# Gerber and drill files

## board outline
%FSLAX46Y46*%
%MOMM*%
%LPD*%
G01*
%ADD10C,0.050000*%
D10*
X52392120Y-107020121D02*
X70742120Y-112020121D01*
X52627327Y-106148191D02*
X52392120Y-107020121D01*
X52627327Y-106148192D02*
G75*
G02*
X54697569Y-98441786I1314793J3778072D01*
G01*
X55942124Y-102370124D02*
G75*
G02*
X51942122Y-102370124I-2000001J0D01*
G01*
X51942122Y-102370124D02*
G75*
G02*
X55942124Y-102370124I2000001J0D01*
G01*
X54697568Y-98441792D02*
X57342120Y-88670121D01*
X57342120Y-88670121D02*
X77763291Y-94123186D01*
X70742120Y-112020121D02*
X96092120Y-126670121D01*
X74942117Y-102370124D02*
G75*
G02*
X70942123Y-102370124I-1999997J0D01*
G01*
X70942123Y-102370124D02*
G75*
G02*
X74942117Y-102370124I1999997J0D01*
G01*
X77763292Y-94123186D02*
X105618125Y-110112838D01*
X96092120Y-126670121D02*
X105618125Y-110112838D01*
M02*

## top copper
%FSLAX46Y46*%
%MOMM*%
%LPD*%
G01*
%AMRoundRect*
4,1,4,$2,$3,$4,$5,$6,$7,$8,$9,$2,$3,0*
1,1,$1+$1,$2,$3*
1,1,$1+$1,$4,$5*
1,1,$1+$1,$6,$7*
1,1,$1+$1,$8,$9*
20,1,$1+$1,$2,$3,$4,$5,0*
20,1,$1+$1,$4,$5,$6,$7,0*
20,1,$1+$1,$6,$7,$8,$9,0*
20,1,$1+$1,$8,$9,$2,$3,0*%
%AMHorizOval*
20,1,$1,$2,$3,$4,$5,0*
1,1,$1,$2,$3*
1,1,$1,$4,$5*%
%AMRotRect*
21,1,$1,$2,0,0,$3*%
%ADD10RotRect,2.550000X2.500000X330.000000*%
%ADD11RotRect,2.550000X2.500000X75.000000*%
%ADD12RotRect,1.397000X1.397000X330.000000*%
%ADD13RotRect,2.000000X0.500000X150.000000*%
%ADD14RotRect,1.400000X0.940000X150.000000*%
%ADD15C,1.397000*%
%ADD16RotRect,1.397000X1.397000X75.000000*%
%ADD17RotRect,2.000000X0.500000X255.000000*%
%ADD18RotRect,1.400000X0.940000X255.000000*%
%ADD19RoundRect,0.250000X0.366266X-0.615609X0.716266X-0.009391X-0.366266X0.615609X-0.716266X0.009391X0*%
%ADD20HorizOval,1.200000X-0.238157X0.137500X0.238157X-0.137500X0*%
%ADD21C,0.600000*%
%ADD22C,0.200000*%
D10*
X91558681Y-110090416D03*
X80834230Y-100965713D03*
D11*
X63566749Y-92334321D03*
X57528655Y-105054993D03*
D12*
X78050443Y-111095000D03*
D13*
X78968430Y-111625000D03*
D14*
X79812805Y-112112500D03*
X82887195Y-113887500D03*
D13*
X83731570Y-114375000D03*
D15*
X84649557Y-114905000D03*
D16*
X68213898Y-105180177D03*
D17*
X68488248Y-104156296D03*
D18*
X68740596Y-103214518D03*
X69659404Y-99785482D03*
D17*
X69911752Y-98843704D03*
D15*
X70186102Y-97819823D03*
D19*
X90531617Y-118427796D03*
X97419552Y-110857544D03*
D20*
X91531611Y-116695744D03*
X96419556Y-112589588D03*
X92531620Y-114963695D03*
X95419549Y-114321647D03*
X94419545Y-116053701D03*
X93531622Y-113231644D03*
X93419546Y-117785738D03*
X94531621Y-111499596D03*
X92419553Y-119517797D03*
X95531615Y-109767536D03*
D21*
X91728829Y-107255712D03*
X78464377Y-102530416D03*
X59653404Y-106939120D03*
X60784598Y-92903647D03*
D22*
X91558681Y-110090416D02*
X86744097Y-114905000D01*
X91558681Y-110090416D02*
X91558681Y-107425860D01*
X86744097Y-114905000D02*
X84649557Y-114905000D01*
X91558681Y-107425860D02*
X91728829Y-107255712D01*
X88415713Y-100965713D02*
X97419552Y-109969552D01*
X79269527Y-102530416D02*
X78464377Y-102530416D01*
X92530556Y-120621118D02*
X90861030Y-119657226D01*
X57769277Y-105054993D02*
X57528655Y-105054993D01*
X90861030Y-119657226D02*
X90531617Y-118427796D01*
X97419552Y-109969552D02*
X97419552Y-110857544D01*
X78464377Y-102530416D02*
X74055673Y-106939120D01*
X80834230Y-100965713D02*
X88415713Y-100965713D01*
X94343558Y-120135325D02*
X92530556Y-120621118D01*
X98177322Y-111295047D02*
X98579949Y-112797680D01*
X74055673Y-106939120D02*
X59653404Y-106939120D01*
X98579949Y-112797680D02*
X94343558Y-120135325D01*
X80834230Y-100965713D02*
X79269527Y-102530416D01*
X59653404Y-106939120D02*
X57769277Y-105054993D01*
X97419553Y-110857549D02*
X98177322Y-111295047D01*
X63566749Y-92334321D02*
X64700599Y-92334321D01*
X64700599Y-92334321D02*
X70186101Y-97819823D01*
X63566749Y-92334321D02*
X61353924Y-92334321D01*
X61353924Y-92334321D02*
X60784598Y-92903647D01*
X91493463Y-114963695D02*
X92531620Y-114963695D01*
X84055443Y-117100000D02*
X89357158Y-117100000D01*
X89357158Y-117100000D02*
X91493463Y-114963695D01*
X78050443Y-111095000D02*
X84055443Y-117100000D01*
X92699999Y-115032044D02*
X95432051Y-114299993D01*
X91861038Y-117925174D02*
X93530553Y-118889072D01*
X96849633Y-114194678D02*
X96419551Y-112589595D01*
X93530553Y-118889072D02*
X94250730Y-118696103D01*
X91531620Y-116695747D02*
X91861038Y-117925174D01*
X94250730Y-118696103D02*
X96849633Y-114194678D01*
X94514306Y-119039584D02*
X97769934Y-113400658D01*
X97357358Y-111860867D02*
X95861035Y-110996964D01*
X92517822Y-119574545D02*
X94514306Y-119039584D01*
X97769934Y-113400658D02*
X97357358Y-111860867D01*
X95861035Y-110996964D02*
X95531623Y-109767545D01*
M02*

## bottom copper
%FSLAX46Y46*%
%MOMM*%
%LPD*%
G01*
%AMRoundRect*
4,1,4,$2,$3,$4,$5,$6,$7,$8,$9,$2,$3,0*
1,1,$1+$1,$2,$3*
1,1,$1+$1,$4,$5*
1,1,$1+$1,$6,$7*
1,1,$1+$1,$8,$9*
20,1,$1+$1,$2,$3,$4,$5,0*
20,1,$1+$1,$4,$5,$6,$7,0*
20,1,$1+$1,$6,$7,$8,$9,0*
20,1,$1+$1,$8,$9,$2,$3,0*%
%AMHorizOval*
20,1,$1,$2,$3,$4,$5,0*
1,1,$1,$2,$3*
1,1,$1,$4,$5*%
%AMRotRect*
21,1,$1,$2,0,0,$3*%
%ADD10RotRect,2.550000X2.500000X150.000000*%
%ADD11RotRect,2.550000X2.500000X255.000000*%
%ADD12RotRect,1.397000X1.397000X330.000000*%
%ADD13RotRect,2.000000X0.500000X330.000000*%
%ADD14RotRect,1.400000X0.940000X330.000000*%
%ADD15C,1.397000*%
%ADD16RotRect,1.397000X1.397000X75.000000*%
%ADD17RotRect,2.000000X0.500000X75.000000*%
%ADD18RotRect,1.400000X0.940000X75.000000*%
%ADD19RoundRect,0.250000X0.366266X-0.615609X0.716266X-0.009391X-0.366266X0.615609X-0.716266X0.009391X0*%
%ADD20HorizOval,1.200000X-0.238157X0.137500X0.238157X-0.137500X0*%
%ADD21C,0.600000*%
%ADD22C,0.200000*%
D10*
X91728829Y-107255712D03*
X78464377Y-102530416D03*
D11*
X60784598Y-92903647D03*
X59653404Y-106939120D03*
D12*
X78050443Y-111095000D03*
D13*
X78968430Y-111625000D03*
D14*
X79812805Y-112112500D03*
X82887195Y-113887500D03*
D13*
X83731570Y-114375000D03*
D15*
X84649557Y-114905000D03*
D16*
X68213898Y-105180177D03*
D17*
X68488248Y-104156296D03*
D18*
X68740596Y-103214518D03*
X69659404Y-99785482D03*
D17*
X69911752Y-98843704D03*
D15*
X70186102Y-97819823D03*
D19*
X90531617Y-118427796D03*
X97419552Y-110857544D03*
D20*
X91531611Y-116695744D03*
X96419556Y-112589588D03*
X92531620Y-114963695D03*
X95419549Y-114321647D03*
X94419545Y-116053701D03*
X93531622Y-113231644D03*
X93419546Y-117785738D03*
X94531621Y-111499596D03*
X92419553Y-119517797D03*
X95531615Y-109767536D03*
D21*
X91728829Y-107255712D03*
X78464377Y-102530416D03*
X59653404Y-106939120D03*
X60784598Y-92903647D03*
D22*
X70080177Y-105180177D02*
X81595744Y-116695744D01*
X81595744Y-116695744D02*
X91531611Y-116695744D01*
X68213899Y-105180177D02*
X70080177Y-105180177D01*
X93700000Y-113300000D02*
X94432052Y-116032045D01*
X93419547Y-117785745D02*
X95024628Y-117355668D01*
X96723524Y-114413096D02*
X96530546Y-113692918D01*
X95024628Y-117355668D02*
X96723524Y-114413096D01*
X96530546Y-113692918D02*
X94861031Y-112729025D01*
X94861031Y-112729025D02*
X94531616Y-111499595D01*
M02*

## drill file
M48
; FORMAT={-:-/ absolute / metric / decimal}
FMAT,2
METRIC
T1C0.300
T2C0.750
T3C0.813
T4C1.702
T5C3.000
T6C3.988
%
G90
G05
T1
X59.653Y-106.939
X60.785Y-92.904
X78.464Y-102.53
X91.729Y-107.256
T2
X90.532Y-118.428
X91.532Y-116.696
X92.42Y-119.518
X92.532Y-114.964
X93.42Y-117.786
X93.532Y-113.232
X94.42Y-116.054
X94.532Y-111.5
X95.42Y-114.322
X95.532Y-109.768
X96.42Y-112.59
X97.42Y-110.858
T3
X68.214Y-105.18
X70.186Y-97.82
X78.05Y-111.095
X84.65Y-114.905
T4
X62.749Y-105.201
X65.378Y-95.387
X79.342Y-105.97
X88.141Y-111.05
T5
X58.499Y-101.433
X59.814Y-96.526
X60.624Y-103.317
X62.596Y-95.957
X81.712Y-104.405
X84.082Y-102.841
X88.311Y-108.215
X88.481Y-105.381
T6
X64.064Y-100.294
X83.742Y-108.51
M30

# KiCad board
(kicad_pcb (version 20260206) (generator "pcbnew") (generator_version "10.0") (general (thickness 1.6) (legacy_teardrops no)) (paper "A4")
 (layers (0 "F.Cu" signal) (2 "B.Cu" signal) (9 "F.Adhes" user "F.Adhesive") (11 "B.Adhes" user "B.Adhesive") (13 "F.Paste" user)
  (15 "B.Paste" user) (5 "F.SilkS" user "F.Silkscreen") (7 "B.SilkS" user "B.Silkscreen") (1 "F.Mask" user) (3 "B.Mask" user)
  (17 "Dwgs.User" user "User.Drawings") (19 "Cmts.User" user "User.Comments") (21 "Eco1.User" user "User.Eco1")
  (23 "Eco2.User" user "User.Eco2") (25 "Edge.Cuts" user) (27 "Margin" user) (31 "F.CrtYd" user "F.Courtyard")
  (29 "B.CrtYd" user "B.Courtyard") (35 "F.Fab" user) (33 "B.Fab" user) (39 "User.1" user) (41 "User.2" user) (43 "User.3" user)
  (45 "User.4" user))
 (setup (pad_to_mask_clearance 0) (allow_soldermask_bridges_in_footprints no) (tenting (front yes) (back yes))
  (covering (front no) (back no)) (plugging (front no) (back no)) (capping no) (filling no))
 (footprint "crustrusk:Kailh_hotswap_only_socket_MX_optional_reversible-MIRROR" (layer "F.Cu") (at 83.741529 108.510121 -30)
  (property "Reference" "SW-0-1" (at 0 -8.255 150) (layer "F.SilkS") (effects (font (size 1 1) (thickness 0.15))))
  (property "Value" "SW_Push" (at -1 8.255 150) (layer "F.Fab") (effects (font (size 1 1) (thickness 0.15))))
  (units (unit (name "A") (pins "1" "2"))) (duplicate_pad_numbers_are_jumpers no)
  (pad "" np_thru_hole circle (at -5.08 0 330) (size 1.7018 1.7018) (drill 1.7018) (layers "*.Cu" "*.Mask"))
  (pad "" np_thru_hole circle (at -3.81 -2.54 150) (size 3 3) (drill 3) (layers "*.Cu" "*.Mask"))
  (pad "" np_thru_hole circle (at -2.54 -5.079997 330) (size 3 3) (drill 3) (layers "*.Cu" "*.Mask"))
  (pad "" np_thru_hole circle (at 0 0 330) (size 3.9878 3.9878) (drill 3.9878) (layers "*.Cu" "*.Mask"))
  (pad "" np_thru_hole circle (at 2.540002 -5.080001 150) (size 3 3) (drill 3) (layers "*.Cu" "*.Mask"))
  (pad "" np_thru_hole circle (at 3.81 -2.540001 330) (size 3 3) (drill 3) (layers "*.Cu" "*.Mask"))
  (pad "" np_thru_hole circle (at 5.08 0 330) (size 1.7018 1.7018) (drill 1.7018) (layers "*.Cu" "*.Mask"))
  (pad "1" smd rect (at 6.29 -5.08 150) (size 2.55 2.5) (layers "B.Cu" "B.Mask" "B.Paste") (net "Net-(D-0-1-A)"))
  (pad "1" smd rect (at 7.56 -2.54 330) (size 2.55 2.5) (layers "F.Cu" "F.Mask" "F.Paste") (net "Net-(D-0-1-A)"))
  (pad "2" smd rect (at -7.56 -2.54 150) (size 2.55 2.5) (layers "B.Cu" "B.Mask" "B.Paste") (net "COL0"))
  (pad "2" smd rect (at -6.289999 -5.079999 330) (size 2.55 2.5) (layers "F.Cu" "F.Mask" "F.Paste") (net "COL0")))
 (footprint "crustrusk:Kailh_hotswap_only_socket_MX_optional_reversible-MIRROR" (layer "F.Cu") (at 64.063529 100.294121 75)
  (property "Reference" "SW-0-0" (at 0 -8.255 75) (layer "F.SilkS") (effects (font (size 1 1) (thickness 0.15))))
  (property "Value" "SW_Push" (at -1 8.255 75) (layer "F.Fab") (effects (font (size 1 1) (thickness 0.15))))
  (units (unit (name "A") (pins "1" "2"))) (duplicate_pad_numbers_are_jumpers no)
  (pad "" np_thru_hole circle (at -5.08 0 75) (size 1.7018 1.7018) (drill 1.7018) (layers "*.Cu" "*.Mask"))
  (pad "" np_thru_hole circle (at -3.810001 -2.54 255) (size 3 3) (drill 3) (layers "*.Cu" "*.Mask"))
  (pad "" np_thru_hole circle (at -2.54 -5.079998 75) (size 3 3) (drill 3) (layers "*.Cu" "*.Mask"))
  (pad "" np_thru_hole circle (at 0 0 75) (size 3.9878 3.9878) (drill 3.9878) (layers "*.Cu" "*.Mask"))
  (pad "" np_thru_hole circle (at 2.540003 -5.080001 255) (size 3 3) (drill 3) (layers "*.Cu" "*.Mask"))
  (pad "" np_thru_hole circle (at 3.81 -2.54 75) (size 3 3) (drill 3) (layers "*.Cu" "*.Mask"))
  (pad "" np_thru_hole circle (at 5.08 0 75) (size 1.7018 1.7018) (drill 1.7018) (layers "*.Cu" "*.Mask"))
  (pad "1" smd rect (at 6.29 -5.08 255) (size 2.55 2.5) (layers "B.Cu" "B.Mask" "B.Paste") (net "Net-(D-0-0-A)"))
  (pad "1" smd rect (at 7.56 -2.54 75) (size 2.55 2.5) (layers "F.Cu" "F.Mask" "F.Paste") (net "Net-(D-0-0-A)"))
  (pad "2" smd rect (at -7.56 -2.540001 255) (size 2.55 2.5) (layers "B.Cu" "B.Mask" "B.Paste") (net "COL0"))
  (pad "2" smd rect (at -6.289999 -5.079999 75) (size 2.55 2.5) (layers "F.Cu" "F.Mask" "F.Paste") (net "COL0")))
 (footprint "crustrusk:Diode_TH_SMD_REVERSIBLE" (layer "F.Cu") (at 81.35 113 -30)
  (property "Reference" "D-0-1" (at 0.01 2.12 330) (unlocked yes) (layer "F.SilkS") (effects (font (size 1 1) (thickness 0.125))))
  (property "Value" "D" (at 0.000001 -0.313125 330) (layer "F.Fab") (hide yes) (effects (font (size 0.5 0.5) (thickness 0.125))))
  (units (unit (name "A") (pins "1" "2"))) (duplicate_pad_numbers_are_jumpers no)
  (pad "1" thru_hole rect (at -3.81 0 330) (size 1.397 1.397) (drill 0.8128) (layers "*.Cu" "*.Mask") (remove_unused_layers no)
   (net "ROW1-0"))
  (pad "1" smd rect (at -2.75 0 150) (size 2 0.5) (layers "F.Cu") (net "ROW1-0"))
  (pad "1" smd rect (at -2.75 0 330) (size 2 0.5) (layers "B.Cu") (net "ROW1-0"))
  (pad "1" smd rect (at -1.775 0 150) (size 1.4 0.94) (layers "F.Cu" "F.Mask" "F.Paste") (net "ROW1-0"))
  (pad "1" smd rect (at -1.775 0 330) (size 1.4 0.94) (layers "B.Cu" "B.Mask" "B.Paste") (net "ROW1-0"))
  (pad "2" smd rect (at 1.775 0 150) (size 1.4 0.94) (layers "F.Cu" "F.Mask" "F.Paste") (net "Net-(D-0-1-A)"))
  (pad "2" smd rect (at 1.775 0 330) (size 1.4 0.94) (layers "B.Cu" "B.Mask" "B.Paste") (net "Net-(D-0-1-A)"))
  (pad "2" smd rect (at 2.75 0 150) (size 2 0.5) (layers "F.Cu") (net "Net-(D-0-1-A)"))
  (pad "2" smd rect (at 2.75 0 330) (size 2 0.5) (layers "B.Cu") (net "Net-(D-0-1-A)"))
  (pad "2" thru_hole circle (at 3.81 0 330) (size 1.397 1.397) (drill 0.8128) (layers "*.Cu" "*.Mask") (remove_unused_layers no)
   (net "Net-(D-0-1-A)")))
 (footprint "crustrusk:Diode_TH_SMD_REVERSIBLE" (layer "F.Cu") (at 69.2 101.5 75)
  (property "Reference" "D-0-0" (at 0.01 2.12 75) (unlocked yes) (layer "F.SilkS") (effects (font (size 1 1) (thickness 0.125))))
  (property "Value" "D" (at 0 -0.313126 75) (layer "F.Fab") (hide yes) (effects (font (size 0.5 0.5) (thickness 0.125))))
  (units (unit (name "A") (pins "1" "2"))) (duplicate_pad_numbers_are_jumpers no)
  (pad "1" thru_hole rect (at -3.81 -0.000001 75) (size 1.397 1.397) (drill 0.8128) (layers "*.Cu" "*.Mask") (remove_unused_layers no)
   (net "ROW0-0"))
  (pad "1" smd rect (at -2.75 0 255) (size 2 0.5) (layers "F.Cu") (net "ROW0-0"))
  (pad "1" smd rect (at -2.75 0 75) (size 2 0.5) (layers "B.Cu") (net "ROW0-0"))
  (pad "1" smd rect (at -1.775 0 255) (size 1.4 0.94) (layers "F.Cu" "F.Mask" "F.Paste") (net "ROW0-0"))
  (pad "1" smd rect (at -1.775 0 75) (size 1.4 0.94) (layers "B.Cu" "B.Mask" "B.Paste") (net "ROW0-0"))
  (pad "2" smd rect (at 1.775 0 255) (size 1.4 0.94) (layers "F.Cu" "F.Mask" "F.Paste") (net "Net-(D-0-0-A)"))
  (pad "2" smd rect (at 1.775 0 75) (size 1.4 0.94) (layers "B.Cu" "B.Mask" "B.Paste") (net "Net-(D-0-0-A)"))
  (pad "2" smd rect (at 2.75 0 255) (size 2 0.5) (layers "F.Cu") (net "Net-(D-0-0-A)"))
  (pad "2" smd rect (at 2.75 0 75) (size 2 0.5) (layers "B.Cu") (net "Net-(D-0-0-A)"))
  (pad "2" thru_hole circle (at 3.81 0.000001 75) (size 1.397 1.397) (drill 0.8128) (layers "*.Cu" "*.Mask") (remove_unused_layers no)
   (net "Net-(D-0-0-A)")))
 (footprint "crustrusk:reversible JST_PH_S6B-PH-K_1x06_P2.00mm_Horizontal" (layer "F.Cu") (at 90.531617 118.427796 60)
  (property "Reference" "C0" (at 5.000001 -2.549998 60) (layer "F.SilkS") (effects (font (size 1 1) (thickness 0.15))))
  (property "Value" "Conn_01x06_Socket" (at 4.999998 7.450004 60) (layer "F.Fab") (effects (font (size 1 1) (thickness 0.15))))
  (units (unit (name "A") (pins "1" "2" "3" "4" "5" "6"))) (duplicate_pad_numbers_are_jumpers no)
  (pad "1" thru_hole roundrect (at 0 0 60) (size 1.2 1.75) (drill 0.75) (layers "*.Cu" "*.Mask") (remove_unused_layers no)
   (roundrect_rratio 0.208333) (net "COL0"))
  (pad "1" thru_hole roundrect (at 9.999998 2.180001 60) (size 1.2 1.75) (drill 0.75) (layers "*.Cu" "*.Mask") (remove_unused_layers no)
   (roundrect_rratio 0.208333) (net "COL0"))
  (pad "2" thru_hole oval (at 1.999998 -0.000006 60) (size 1.2 1.75) (drill 0.75) (layers "*.Cu" "*.Mask") (remove_unused_layers no)
   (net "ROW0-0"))
  (pad "2" thru_hole oval (at 8.000006 2.180001 60) (size 1.2 1.75) (drill 0.75) (layers "*.Cu" "*.Mask") (remove_unused_layers no)
   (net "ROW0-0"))
  (pad "3" thru_hole oval (at 4.000001 0.000003 60) (size 1.2 1.75) (drill 0.75) (layers "*.Cu" "*.Mask") (remove_unused_layers no)
   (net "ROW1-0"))
  (pad "3" thru_hole oval (at 5.999995 2.179999 60) (size 1.2 1.75) (drill 0.75) (layers "*.Cu" "*.Mask") (remove_unused_layers no)
   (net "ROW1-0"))
  (pad "4" thru_hole oval (at 3.999991 2.179997 60) (size 1.2 1.75) (drill 0.75) (layers "*.Cu" "*.Mask") (remove_unused_layers no)
   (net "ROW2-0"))
  (pad "4" thru_hole oval (at 6.000002 0.000005 60) (size 1.2 1.75) (drill 0.75) (layers "*.Cu" "*.Mask") (remove_unused_layers no)
   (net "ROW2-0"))
  (pad "5" thru_hole oval (at 2.000003 2.179991 60) (size 1.2 1.75) (drill 0.75) (layers "*.Cu" "*.Mask") (remove_unused_layers no)
   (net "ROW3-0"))
  (pad "5" thru_hole oval (at 7.999999 0.000005 60) (size 1.2 1.75) (drill 0.75) (layers "*.Cu" "*.Mask") (remove_unused_layers no)
   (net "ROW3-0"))
  (pad "6" thru_hole oval (at -0.000001 2.180001 60) (size 1.2 1.75) (drill 0.75) (layers "*.Cu" "*.Mask") (remove_unused_layers no)
   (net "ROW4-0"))
  (pad "6" thru_hole oval (at 10.000004 -0.000005 60) (size 1.2 1.75) (drill 0.75) (layers "*.Cu" "*.Mask") (remove_unused_layers no)
   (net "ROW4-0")))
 (gr_line (start 52.39212 107.020121) (end 70.74212 112.020121) (stroke (width 0.05) (type default)) (layer "Edge.Cuts"))
 (gr_line (start 52.627327 106.148191) (end 52.39212 107.020121) (stroke (width 0.05) (type default)) (layer "Edge.Cuts"))
 (gr_arc (start 52.627327 106.148192) (mid 50.078787 101.33228) (end 54.697568 98.441792) (stroke (width 0.05) (type default))
  (layer "Edge.Cuts"))
 (gr_circle (center 53.942123 102.370124) (end 51.942122 102.370124) (stroke (width 0.05) (type default)) (fill no) (layer "Edge.Cuts"))
 (gr_line (start 54.697568 98.441792) (end 57.34212 88.670121) (stroke (width 0.05) (type default)) (layer "Edge.Cuts"))
 (gr_line (start 57.34212 88.670121) (end 77.763291 94.123186) (stroke (width 0.05) (type default)) (layer "Edge.Cuts"))
 (gr_line (start 70.74212 112.020121) (end 96.09212 126.670121) (stroke (width 0.05) (type default)) (layer "Edge.Cuts"))
 (gr_circle (center 72.94212 102.370124) (end 70.942123 102.370124) (stroke (width 0.05) (type default)) (fill no) (layer "Edge.Cuts"))
 (gr_line (start 77.763292 94.123186) (end 105.618125 110.112838) (stroke (width 0.05) (type default)) (layer "Edge.Cuts"))
 (gr_line (start 96.09212 126.670121) (end 105.618125 110.112838) (stroke (width 0.05) (type default)) (layer "Edge.Cuts"))
 (segment (start 91.558681 110.090416) (end 86.744097 114.905) (width 0.2) (layer "F.Cu") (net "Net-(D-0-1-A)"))
 (segment (start 91.558681 110.090416) (end 91.558681 107.42586) (width 0.2) (layer "F.Cu") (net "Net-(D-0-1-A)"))
 (segment (start 86.744097 114.905) (end 84.649557 114.905) (width 0.2) (layer "F.Cu") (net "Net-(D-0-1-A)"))
 (segment (start 91.558681 107.42586) (end 91.728829 107.255712) (width 0.2) (layer "F.Cu") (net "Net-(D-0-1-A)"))
 (via (at 91.728829 107.255712) (size 0.6) (drill 0.3) (layers "F.Cu" "B.Cu") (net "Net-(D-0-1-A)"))
 (segment (start 88.415713 100.965713) (end 97.419552 109.969552) (width 0.2) (layer "F.Cu") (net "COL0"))
 (segment (start 79.269527 102.530416) (end 78.464377 102.530416) (width 0.2) (layer "F.Cu") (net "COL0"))
 (segment (start 92.530556 120.621118) (end 90.86103 119.657226) (width 0.2) (layer "F.Cu") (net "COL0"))
 (segment (start 57.769277 105.054993) (end 57.528655 105.054993) (width 0.2) (layer "F.Cu") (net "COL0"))
 (segment (start 90.86103 119.657226) (end 90.531617 118.427796) (width 0.2) (layer "F.Cu") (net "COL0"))
 (segment (start 97.419552 109.969552) (end 97.419552 110.857544) (width 0.2) (layer "F.Cu") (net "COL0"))
 (segment (start 78.464377 102.530416) (end 74.055673 106.93912) (width 0.2) (layer "F.Cu") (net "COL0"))
 (segment (start 80.83423 100.965713) (end 88.415713 100.965713) (width 0.2) (layer "F.Cu") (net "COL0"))
 (segment (start 94.343558 120.135325) (end 92.530556 120.621118) (width 0.2) (layer "F.Cu") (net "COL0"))
 (segment (start 98.177322 111.295047) (end 98.579949 112.79768) (width 0.2) (layer "F.Cu") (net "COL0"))
 (segment (start 74.055673 106.93912) (end 59.653404 106.93912) (width 0.2) (layer "F.Cu") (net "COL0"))
 (segment (start 98.579949 112.79768) (end 94.343558 120.135325) (width 0.2) (layer "F.Cu") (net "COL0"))
 (segment (start 80.83423 100.965713) (end 79.269527 102.530416) (width 0.2) (layer "F.Cu") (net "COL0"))
 (segment (start 59.653404 106.93912) (end 57.769277 105.054993) (width 0.2) (layer "F.Cu") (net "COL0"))
 (segment (start 97.419553 110.857549) (end 98.177322 111.295047) (width 0.2) (layer "F.Cu") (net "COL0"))
 (via (at 78.464377 102.530416) (size 0.6) (drill 0.3) (layers "F.Cu" "B.Cu") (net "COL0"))
 (via (at 59.653404 106.93912) (size 0.6) (drill 0.3) (layers "F.Cu" "B.Cu") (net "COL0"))
 (segment (start 63.566749 92.334321) (end 64.700599 92.334321) (width 0.2) (layer "F.Cu") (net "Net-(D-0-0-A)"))
 (segment (start 64.700599 92.334321) (end 70.186101 97.819823) (width 0.2) (layer "F.Cu") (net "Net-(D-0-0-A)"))
 (segment (start 63.566749 92.334321) (end 61.353924 92.334321) (width 0.2) (layer "F.Cu") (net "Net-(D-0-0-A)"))
 (segment (start 61.353924 92.334321) (end 60.784598 92.903647) (width 0.2) (layer "F.Cu") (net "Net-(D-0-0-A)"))
 (via (at 60.784598 92.903647) (size 0.6) (drill 0.3) (layers "F.Cu" "B.Cu") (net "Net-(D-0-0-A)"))
 (segment (start 91.493463 114.963695) (end 92.53162 114.963695) (width 0.2) (layer "F.Cu") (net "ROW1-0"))
 (segment (start 84.055443 117.1) (end 89.357158 117.1) (width 0.2) (layer "F.Cu") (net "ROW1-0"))
 (segment (start 89.357158 117.1) (end 91.493463 114.963695) (width 0.2) (layer "F.Cu") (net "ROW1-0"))
 (segment (start 78.050443 111.095) (end 84.055443 117.1) (width 0.2) (layer "F.Cu") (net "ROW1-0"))
 (segment (start 92.699999 115.032044) (end 95.432051 114.299993) (width 0.2) (layer "F.Cu") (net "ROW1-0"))
 (segment (start 91.861038 117.925174) (end 93.530553 118.889072) (width 0.2) (layer "F.Cu") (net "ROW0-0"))
 (segment (start 96.849633 114.194678) (end 96.419551 112.589595) (width 0.2) (layer "F.Cu") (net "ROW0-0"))
 (segment (start 93.530553 118.889072) (end 94.25073 118.696103) (width 0.2) (layer "F.Cu") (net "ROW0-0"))
 (segment (start 91.53162 116.695747) (end 91.861038 117.925174) (width 0.2) (layer "F.Cu") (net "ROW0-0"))
 (segment (start 94.25073 118.696103) (end 96.849633 114.194678) (width 0.2) (layer "F.Cu") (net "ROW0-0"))
 (segment (start 70.080177 105.180177) (end 81.595744 116.695744) (width 0.2) (layer "B.Cu") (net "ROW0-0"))
 (segment (start 81.595744 116.695744) (end 91.531611 116.695744) (width 0.2) (layer "B.Cu") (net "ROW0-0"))
 (segment (start 68.213899 105.180177) (end 70.080177 105.180177) (width 0.2) (layer "B.Cu") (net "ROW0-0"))
 (segment (start 93.7 113.3) (end 94.432052 116.032045) (width 0.2) (layer "B.Cu") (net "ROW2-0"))
 (segment (start 93.419547 117.785745) (end 95.024628 117.355668) (width 0.2) (layer "B.Cu") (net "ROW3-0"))
 (segment (start 96.723524 114.413096) (end 96.530546 113.692918) (width 0.2) (layer "B.Cu") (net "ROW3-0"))
 (segment (start 95.024628 117.355668) (end 96.723524 114.413096) (width 0.2) (layer "B.Cu") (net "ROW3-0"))
 (segment (start 96.530546 113.692918) (end 94.861031 112.729025) (width 0.2) (layer "B.Cu") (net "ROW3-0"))
 (segment (start 94.861031 112.729025) (end 94.531616 111.499595) (width 0.2) (layer "B.Cu") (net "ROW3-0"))
 (segment (start 94.514306 119.039584) (end 97.769934 113.400658) (width 0.2) (layer "F.Cu") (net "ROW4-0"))
 (segment (start 97.357358 111.860867) (end 95.861035 110.996964) (width 0.2) (layer "F.Cu") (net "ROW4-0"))
 (segment (start 92.517822 119.574545) (end 94.514306 119.039584) (width 0.2) (layer "F.Cu") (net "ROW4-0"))
 (segment (start 97.769934 113.400658) (end 97.357358 111.860867) (width 0.2) (layer "F.Cu") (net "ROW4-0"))
 (segment (start 95.861035 110.996964) (end 95.531623 109.767545) (width 0.2) (layer "F.Cu") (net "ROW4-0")))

